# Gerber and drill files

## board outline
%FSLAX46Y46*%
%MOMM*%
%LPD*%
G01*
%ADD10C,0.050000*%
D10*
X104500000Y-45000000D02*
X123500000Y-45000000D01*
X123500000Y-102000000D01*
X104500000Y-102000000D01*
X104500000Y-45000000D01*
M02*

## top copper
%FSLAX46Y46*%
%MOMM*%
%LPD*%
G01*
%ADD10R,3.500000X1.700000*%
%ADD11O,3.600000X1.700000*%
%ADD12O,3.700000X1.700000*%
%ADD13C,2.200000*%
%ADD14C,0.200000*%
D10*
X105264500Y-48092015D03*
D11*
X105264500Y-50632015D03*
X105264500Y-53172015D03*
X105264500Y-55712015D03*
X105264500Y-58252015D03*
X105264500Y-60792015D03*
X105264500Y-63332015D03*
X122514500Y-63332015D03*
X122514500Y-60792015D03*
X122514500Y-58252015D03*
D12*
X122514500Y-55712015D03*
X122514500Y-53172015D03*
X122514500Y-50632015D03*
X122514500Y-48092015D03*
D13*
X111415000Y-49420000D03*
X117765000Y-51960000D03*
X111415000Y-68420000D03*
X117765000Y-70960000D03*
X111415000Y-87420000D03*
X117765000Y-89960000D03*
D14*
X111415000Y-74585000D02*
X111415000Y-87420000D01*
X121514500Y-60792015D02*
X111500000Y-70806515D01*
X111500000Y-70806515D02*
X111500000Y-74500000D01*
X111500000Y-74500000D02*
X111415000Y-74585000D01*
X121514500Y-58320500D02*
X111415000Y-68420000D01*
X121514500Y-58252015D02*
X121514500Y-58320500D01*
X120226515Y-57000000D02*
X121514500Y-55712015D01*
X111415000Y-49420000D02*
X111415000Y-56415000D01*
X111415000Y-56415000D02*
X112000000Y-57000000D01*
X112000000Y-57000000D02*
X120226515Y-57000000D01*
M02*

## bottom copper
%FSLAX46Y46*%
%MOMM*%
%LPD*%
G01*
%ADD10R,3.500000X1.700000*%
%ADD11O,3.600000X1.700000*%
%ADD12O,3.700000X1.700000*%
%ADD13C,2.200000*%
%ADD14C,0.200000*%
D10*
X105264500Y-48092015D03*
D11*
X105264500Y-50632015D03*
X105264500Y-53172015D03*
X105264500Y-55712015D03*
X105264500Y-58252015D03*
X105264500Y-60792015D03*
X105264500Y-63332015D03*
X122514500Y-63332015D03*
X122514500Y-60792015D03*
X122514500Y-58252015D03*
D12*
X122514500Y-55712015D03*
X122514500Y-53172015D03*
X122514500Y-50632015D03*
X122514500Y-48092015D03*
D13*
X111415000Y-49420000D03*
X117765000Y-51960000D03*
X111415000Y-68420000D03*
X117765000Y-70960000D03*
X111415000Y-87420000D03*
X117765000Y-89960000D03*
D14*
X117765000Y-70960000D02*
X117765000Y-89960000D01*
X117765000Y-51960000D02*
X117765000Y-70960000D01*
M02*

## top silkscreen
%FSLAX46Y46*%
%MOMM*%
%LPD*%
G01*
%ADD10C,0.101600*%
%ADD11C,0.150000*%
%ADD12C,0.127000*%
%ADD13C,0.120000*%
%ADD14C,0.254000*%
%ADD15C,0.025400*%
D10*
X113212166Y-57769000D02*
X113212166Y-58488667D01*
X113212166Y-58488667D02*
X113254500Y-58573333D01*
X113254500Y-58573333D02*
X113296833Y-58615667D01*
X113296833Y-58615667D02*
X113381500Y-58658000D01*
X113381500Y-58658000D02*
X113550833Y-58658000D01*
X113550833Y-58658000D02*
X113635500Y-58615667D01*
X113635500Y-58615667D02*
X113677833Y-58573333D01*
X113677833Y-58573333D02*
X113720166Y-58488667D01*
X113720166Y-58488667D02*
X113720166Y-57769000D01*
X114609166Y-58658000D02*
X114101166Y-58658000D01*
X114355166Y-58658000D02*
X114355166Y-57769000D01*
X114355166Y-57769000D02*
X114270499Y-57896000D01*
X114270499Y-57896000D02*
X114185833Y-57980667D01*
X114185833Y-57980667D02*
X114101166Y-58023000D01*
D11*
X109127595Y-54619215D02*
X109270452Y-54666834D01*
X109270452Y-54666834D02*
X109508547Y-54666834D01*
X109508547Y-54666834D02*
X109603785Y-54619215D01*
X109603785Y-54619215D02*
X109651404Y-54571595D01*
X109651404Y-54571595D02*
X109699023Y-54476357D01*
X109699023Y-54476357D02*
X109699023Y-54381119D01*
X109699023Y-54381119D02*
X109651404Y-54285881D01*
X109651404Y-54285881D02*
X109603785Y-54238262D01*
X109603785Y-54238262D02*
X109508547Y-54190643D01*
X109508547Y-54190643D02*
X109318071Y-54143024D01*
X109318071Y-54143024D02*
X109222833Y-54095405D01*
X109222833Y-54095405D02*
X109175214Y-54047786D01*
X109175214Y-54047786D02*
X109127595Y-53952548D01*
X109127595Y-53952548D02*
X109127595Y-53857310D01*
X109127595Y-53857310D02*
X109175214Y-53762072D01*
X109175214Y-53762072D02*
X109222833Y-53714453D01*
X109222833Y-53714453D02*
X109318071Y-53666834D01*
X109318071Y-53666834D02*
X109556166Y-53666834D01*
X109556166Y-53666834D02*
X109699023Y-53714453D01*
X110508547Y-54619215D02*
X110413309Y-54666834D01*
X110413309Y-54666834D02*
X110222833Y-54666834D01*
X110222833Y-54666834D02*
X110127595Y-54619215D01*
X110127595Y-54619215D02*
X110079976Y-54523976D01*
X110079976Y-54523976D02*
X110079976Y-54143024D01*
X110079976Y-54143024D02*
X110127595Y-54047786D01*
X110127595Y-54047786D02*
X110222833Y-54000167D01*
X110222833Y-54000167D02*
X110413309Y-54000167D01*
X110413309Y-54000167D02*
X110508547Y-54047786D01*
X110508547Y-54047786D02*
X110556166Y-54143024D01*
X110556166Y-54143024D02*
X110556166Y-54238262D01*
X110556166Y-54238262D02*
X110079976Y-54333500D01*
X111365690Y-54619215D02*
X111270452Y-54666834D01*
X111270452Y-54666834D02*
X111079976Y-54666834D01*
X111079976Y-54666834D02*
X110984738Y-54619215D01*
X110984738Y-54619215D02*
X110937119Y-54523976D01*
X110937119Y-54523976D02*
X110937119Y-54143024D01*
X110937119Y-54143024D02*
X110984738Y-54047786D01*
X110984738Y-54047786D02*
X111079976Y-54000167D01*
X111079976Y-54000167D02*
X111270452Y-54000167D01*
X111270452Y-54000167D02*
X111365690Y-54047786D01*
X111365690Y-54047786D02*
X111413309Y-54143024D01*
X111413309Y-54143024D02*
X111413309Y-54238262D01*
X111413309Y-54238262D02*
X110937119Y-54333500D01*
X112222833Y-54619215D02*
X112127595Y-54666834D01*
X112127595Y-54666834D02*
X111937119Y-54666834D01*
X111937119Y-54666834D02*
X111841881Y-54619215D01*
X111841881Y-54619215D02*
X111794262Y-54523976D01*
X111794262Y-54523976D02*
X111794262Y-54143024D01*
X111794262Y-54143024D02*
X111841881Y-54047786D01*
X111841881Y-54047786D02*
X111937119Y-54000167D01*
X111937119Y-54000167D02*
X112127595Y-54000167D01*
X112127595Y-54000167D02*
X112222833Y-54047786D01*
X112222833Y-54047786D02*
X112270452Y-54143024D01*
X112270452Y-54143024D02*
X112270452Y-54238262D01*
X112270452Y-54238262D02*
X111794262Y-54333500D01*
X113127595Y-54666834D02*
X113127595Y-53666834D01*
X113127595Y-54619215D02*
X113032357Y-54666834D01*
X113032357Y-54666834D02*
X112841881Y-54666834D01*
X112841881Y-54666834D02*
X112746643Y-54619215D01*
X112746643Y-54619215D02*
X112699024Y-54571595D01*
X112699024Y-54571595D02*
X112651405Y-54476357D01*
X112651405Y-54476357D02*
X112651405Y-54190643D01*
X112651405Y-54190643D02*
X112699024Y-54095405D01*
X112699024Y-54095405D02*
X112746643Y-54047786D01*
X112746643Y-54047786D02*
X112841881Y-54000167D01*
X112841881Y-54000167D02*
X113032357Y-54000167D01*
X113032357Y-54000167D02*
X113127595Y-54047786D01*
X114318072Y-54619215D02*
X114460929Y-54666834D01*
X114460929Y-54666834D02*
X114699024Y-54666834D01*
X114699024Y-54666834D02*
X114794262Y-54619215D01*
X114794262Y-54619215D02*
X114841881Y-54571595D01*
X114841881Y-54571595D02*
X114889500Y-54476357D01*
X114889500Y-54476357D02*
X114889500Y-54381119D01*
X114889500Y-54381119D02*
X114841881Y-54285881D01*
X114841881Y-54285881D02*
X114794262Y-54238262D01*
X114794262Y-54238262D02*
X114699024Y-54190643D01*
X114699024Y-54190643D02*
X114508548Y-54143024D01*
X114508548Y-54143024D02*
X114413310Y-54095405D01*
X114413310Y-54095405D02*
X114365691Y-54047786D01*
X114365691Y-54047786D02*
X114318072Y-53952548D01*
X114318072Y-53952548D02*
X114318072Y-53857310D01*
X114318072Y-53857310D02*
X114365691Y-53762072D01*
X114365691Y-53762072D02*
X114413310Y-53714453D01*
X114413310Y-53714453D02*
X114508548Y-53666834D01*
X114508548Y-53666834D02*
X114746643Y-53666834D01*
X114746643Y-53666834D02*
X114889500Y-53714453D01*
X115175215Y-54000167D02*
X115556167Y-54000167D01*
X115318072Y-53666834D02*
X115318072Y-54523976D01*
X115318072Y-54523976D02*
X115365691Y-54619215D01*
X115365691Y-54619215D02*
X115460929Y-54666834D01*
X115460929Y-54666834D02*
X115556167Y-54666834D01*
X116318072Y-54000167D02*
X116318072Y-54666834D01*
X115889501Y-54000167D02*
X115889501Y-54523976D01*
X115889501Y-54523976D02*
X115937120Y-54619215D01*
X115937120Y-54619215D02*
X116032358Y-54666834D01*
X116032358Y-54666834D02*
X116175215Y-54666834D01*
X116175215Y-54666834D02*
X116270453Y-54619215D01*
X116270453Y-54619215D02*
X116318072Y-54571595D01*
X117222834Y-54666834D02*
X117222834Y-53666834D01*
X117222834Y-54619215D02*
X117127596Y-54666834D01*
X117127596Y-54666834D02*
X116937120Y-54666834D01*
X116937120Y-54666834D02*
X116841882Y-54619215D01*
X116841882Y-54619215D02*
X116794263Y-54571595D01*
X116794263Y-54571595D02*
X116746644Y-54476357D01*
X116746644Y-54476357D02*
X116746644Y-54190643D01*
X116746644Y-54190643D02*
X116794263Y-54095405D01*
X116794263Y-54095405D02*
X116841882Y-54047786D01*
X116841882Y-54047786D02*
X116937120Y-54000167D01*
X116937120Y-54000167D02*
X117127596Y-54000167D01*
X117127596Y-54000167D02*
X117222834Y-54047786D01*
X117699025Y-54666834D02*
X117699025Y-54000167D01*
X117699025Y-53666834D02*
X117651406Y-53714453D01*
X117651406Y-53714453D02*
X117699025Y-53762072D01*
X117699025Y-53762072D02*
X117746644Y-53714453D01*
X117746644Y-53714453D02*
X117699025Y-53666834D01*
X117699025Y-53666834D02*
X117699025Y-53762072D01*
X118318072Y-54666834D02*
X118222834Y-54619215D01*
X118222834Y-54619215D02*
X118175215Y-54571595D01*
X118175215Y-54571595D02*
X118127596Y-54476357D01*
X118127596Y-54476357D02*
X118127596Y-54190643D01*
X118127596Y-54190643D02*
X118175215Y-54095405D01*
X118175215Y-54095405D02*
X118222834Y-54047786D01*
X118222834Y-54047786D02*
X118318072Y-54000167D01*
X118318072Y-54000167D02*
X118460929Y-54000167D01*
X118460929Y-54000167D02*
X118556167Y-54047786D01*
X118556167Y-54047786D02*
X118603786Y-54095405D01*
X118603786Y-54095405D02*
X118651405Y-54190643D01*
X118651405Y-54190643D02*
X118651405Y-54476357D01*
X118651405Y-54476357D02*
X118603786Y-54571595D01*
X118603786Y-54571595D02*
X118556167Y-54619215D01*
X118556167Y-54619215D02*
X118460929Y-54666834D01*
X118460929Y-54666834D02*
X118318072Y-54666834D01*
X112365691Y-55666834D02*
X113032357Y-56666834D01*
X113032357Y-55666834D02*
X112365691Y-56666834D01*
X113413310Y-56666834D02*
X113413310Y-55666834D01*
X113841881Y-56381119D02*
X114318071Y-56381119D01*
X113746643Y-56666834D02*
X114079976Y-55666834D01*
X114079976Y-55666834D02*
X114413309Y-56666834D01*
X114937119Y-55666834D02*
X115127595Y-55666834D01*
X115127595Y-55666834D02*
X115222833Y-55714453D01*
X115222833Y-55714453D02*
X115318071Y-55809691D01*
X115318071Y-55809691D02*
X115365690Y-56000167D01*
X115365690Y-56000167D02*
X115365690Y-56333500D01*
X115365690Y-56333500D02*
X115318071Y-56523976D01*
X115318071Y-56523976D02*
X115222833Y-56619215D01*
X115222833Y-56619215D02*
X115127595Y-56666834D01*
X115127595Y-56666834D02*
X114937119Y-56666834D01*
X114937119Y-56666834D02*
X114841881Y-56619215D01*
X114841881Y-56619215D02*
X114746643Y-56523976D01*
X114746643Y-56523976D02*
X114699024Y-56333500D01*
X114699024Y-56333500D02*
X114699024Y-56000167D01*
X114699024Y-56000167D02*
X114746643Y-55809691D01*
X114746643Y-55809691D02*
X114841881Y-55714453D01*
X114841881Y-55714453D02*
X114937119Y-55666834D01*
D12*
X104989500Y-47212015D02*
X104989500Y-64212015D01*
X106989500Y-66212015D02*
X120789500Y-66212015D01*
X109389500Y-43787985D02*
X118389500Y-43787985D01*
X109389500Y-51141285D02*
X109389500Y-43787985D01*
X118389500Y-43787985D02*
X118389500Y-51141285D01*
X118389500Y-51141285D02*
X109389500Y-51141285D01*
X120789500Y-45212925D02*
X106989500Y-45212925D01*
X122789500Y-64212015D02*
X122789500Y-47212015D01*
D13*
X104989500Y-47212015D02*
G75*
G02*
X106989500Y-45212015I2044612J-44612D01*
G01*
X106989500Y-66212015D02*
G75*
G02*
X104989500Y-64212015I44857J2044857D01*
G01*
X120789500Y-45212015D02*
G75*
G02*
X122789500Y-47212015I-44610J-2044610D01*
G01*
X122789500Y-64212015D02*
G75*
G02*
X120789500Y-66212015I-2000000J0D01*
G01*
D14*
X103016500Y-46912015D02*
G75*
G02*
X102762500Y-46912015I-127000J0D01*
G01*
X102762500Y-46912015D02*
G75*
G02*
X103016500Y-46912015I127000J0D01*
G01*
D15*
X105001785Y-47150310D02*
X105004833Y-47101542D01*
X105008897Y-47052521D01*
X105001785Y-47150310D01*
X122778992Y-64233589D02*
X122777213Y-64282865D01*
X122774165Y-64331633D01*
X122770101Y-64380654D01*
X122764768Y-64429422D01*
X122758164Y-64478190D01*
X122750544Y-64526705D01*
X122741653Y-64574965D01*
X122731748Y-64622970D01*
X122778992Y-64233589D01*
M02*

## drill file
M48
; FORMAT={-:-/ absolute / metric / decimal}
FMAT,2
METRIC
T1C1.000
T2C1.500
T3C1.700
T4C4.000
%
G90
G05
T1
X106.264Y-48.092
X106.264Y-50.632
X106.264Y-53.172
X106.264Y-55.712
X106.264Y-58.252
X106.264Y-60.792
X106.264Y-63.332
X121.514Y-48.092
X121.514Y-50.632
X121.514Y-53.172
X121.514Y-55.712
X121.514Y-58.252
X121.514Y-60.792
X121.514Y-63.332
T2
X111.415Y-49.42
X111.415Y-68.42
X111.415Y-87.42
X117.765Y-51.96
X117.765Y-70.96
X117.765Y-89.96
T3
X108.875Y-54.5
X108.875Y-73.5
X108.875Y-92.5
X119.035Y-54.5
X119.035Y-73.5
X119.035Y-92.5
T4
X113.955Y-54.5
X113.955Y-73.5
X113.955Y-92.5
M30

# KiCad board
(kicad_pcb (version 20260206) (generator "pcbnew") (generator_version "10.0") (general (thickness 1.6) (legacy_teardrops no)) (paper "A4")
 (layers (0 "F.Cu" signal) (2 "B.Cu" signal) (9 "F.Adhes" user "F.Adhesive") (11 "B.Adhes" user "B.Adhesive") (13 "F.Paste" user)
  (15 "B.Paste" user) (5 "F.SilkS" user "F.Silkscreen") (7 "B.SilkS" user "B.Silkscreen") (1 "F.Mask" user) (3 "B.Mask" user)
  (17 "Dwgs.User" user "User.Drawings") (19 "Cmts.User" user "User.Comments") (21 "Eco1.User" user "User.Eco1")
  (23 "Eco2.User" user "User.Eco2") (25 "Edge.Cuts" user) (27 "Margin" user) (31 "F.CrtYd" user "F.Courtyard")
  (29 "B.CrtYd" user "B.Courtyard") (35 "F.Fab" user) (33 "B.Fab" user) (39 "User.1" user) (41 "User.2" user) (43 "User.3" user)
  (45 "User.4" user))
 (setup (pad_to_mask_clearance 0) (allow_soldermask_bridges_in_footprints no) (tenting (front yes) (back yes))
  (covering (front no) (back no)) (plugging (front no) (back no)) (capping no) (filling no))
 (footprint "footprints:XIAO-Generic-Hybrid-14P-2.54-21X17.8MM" (layer "F.Cu") (at 113.8895 55.712015)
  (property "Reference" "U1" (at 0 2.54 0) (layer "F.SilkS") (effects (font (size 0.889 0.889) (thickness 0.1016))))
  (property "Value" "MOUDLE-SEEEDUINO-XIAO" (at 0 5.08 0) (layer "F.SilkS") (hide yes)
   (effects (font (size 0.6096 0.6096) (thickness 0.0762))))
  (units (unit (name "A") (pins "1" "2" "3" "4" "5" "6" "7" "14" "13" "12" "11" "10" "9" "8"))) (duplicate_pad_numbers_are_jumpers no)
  (fp_line (start -8.9 -8.5) (end -8.9 8.5) (stroke (width 0.127) (type solid)) (layer "F.SilkS"))
  (fp_line (start -6.9 10.5) (end 6.9 10.5) (stroke (width 0.127) (type solid)) (layer "F.SilkS"))
  (fp_line (start -4.5 -11.92403) (end 4.5 -11.92403) (stroke (width 0.127) (type solid)) (layer "F.SilkS"))
  (fp_line (start -4.5 -4.57073) (end -4.5 -11.92403) (stroke (width 0.127) (type solid)) (layer "F.SilkS"))
  (fp_line (start 4.5 -11.92403) (end 4.5 -4.57073) (stroke (width 0.127) (type solid)) (layer "F.SilkS"))
  (fp_line (start 4.5 -4.57073) (end -4.5 -4.57073) (stroke (width 0.127) (type solid)) (layer "F.SilkS"))
  (fp_line (start 6.9 -10.49909) (end -6.9 -10.49909) (stroke (width 0.127) (type solid)) (layer "F.SilkS"))
  (fp_line (start 8.9 8.5) (end 8.9 -8.5) (stroke (width 0.127) (type solid)) (layer "F.SilkS"))
  (fp_arc (start -8.9 -8.5) (mid -8.301491 -9.901491) (end -6.9 -10.5) (stroke (width 0.12) (type solid)) (layer "F.SilkS"))
  (fp_arc (start -6.9 10.5) (mid -8.301423 9.901423) (end -8.9 8.5) (stroke (width 0.12) (type solid)) (layer "F.SilkS"))
  (fp_arc (start 6.9 -10.5) (mid 8.301491 -9.901491) (end 8.9 -8.5) (stroke (width 0.12) (type solid)) (layer "F.SilkS"))
  (fp_arc (start 8.9 8.5) (mid 8.314214 9.914214) (end 6.9 10.5) (stroke (width 0.12) (type solid)) (layer "F.SilkS"))
  (fp_circle (center -11 -8.8) (end -11 -9.054) (stroke (width 0) (type solid)) (fill yes) (layer "F.SilkS"))
  (fp_poly
   (pts (xy -8.887715 -8.561705) (xy -8.884667 -8.610473) (xy -8.880603 -8.659494)) (stroke (width 0.0254) (type solid)) (fill no)
   (layer "F.SilkS"))
  (fp_poly
   (pts (xy 8.889492 8.521574) (xy 8.887713 8.57085) (xy 8.884665 8.619618) (xy 8.880601 8.668639) (xy 8.875268 8.717407)
    (xy 8.868664 8.766175) (xy 8.861044 8.81469) (xy 8.852153 8.86295) (xy 8.842248 8.910955))
   (stroke (width 0.0254) (type solid)) (fill no) (layer "F.SilkS"))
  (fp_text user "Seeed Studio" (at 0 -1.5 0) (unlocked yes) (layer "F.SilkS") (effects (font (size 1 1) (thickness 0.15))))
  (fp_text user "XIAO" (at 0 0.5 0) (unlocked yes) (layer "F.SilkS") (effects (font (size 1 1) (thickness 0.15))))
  (pad "1" thru_hole rect (at -7.625 -7.62) (size 3.5 1.7) (drill 1 (offset -1 0)) (layers "*.Cu" "*.Mask") (remove_unused_layers no)
   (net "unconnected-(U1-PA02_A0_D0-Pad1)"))
  (pad "2" thru_hole oval (at -7.625 -5.08) (size 3.6 1.7) (drill 1 (offset -1 0)) (layers "*.Cu" "*.Mask") (remove_unused_layers no)
   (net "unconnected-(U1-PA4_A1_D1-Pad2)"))
  (pad "3" thru_hole oval (at -7.625 -2.54) (size 3.6 1.7) (drill 1 (offset -1 0)) (layers "*.Cu" "*.Mask") (remove_unused_layers no)
   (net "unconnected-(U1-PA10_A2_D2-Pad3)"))
  (pad "4" thru_hole oval (at -7.625 0) (size 3.6 1.7) (drill 1 (offset -1 0)) (layers "*.Cu" "*.Mask") (remove_unused_layers no)
   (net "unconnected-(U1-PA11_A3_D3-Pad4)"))
  (pad "5" thru_hole oval (at -7.625 2.54) (size 3.6 1.7) (drill 1 (offset -1 0)) (layers "*.Cu" "*.Mask") (remove_unused_layers no)
   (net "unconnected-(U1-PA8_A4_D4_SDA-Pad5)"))
  (pad "6" thru_hole oval (at -7.625 5.08 180) (size 3.6 1.7) (drill 1 (offset 1 0)) (layers "*.Cu" "*.Mask") (remove_unused_layers no)
   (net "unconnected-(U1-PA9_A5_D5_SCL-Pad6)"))
  (pad "7" thru_hole oval (at -7.625 7.62) (size 3.6 1.7) (drill 1 (offset -1 0)) (layers "*.Cu" "*.Mask") (remove_unused_layers no)
   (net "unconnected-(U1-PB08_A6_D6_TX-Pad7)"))
  (pad "8" thru_hole oval (at 7.625 7.62) (size 3.6 1.7) (drill 1 (offset 1 0)) (layers "*.Cu" "*.Mask") (remove_unused_layers no)
   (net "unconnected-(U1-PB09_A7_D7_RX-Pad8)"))
  (pad "9" thru_hole oval (at 7.625 5.08) (size 3.6 1.7) (drill 1 (offset 1 0)) (layers "*.Cu" "*.Mask") (remove_unused_layers no)
   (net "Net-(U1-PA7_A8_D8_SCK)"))
  (pad "10" thru_hole oval (at 7.625 2.54) (size 3.6 1.7) (drill 1 (offset 1 0)) (layers "*.Cu" "*.Mask") (remove_unused_layers no)
   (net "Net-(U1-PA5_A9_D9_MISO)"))
  (pad "11" thru_hole oval (at 7.625 0) (size 3.7 1.7) (drill 1 (offset 1 0)) (layers "*.Cu" "*.Mask") (remove_unused_layers no)
   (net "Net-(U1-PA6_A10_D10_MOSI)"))
  (pad "12" thru_hole oval (at 7.625 -2.54) (size 3.7 1.7) (drill 1 (offset 1 0)) (layers "*.Cu" "*.Mask") (remove_unused_layers no)
   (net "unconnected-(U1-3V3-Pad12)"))
  (pad "13" thru_hole oval (at 7.625 -5.08) (size 3.7 1.7) (drill 1 (offset 1 0)) (layers "*.Cu" "*.Mask") (remove_unused_layers no)
   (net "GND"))
  (pad "14" thru_hole oval (at 7.625 -7.62) (size 3.7 1.7) (drill 1 (offset 1 0)) (layers "*.Cu" "*.Mask") (remove_unused_layers no)
   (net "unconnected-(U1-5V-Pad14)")))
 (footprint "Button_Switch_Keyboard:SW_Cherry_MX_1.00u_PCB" (layer "B.Cu") (at 111.415 49.42 180)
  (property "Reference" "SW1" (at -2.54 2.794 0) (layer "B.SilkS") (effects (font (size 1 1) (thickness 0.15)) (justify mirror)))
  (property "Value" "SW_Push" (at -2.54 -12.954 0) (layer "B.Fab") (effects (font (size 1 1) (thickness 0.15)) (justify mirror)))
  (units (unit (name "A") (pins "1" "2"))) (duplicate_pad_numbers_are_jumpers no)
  (pad "" np_thru_hole circle (at -7.62 -5.08 180) (size 1.7 1.7) (drill 1.7) (layers "*.Cu" "*.Mask"))
  (pad "" np_thru_hole circle (at -2.54 -5.08 180) (size 4 4) (drill 4) (layers "*.Cu" "*.Mask"))
  (pad "" np_thru_hole circle (at 2.54 -5.08 180) (size 1.7 1.7) (drill 1.7) (layers "*.Cu" "*.Mask"))
  (pad "1" thru_hole circle (at 0 0 180) (size 2.2 2.2) (drill 1.5) (layers "*.Cu" "*.Mask") (remove_unused_layers no)
   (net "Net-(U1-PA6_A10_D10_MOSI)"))
  (pad "2" thru_hole circle (at -6.35 -2.54 180) (size 2.2 2.2) (drill 1.5) (layers "*.Cu" "*.Mask") (remove_unused_layers no) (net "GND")))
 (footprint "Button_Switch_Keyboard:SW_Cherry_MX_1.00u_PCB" (layer "B.Cu") (at 111.415 68.42 180)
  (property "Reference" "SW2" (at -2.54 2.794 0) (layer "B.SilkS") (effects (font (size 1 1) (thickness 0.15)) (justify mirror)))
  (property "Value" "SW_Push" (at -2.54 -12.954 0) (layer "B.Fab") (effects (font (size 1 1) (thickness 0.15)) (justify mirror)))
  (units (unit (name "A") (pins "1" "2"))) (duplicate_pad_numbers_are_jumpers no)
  (pad "" np_thru_hole circle (at -7.62 -5.08 180) (size 1.7 1.7) (drill 1.7) (layers "*.Cu" "*.Mask"))
  (pad "" np_thru_hole circle (at -2.54 -5.08 180) (size 4 4) (drill 4) (layers "*.Cu" "*.Mask"))
  (pad "" np_thru_hole circle (at 2.54 -5.08 180) (size 1.7 1.7) (drill 1.7) (layers "*.Cu" "*.Mask"))
  (pad "1" thru_hole circle (at 0 0 180) (size 2.2 2.2) (drill 1.5) (layers "*.Cu" "*.Mask") (remove_unused_layers no)
   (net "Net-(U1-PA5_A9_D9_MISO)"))
  (pad "2" thru_hole circle (at -6.35 -2.54 180) (size 2.2 2.2) (drill 1.5) (layers "*.Cu" "*.Mask") (remove_unused_layers no) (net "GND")))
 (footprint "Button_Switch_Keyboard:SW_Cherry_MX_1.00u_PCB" (layer "B.Cu") (at 111.415 87.42 180)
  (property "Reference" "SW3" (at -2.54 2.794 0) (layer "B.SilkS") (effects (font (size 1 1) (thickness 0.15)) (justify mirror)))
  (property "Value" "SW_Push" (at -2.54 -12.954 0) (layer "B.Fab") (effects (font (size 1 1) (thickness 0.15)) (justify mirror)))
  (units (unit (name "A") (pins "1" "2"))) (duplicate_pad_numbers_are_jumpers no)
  (pad "" np_thru_hole circle (at -7.62 -5.08 180) (size 1.7 1.7) (drill 1.7) (layers "*.Cu" "*.Mask"))
  (pad "" np_thru_hole circle (at -2.54 -5.08 180) (size 4 4) (drill 4) (layers "*.Cu" "*.Mask"))
  (pad "" np_thru_hole circle (at 2.54 -5.08 180) (size 1.7 1.7) (drill 1.7) (layers "*.Cu" "*.Mask"))
  (pad "1" thru_hole circle (at 0 0 180) (size 2.2 2.2) (drill 1.5) (layers "*.Cu" "*.Mask") (remove_unused_layers no)
   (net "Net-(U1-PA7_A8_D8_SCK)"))
  (pad "2" thru_hole circle (at -6.35 -2.54 180) (size 2.2 2.2) (drill 1.5) (layers "*.Cu" "*.Mask") (remove_unused_layers no) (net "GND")))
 (gr_rect (start 104.5 45) (end 123.5 102) (stroke (width 0.05) (type default)) (fill no) (layer "Edge.Cuts"))
 (segment (start 111.415 74.585) (end 111.415 87.42) (width 0.2) (layer "F.Cu") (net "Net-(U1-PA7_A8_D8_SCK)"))
 (segment (start 121.5145 60.792015) (end 111.5 70.806515) (width 0.2) (layer "F.Cu") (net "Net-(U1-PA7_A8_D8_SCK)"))
 (segment (start 111.5 70.806515) (end 111.5 74.5) (width 0.2) (layer "F.Cu") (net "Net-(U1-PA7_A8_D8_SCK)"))
 (segment (start 111.5 74.5) (end 111.415 74.585) (width 0.2) (layer "F.Cu") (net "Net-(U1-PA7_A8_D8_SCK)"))
 (segment (start 121.5145 58.3205) (end 111.415 68.42) (width 0.2) (layer "F.Cu") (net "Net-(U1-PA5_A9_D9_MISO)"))
 (segment (start 121.5145 58.252015) (end 121.5145 58.3205) (width 0.2) (layer "F.Cu") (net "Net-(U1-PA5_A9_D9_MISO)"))
 (segment (start 120.226515 57) (end 121.5145 55.712015) (width 0.2) (layer "F.Cu") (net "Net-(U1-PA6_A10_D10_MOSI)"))
 (segment (start 111.415 49.42) (end 111.415 56.415) (width 0.2) (layer "F.Cu") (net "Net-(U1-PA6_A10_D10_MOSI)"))
 (segment (start 111.415 56.415) (end 112 57) (width 0.2) (layer "F.Cu") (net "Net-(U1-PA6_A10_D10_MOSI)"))
 (segment (start 112 57) (end 120.226515 57) (width 0.2) (layer "F.Cu") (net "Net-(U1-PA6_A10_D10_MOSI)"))
 (segment (start 117.765 70.96) (end 117.765 89.96) (width 0.2) (layer "B.Cu") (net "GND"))
 (segment (start 117.765 51.96) (end 117.765 70.96) (width 0.2) (layer "B.Cu") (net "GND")))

